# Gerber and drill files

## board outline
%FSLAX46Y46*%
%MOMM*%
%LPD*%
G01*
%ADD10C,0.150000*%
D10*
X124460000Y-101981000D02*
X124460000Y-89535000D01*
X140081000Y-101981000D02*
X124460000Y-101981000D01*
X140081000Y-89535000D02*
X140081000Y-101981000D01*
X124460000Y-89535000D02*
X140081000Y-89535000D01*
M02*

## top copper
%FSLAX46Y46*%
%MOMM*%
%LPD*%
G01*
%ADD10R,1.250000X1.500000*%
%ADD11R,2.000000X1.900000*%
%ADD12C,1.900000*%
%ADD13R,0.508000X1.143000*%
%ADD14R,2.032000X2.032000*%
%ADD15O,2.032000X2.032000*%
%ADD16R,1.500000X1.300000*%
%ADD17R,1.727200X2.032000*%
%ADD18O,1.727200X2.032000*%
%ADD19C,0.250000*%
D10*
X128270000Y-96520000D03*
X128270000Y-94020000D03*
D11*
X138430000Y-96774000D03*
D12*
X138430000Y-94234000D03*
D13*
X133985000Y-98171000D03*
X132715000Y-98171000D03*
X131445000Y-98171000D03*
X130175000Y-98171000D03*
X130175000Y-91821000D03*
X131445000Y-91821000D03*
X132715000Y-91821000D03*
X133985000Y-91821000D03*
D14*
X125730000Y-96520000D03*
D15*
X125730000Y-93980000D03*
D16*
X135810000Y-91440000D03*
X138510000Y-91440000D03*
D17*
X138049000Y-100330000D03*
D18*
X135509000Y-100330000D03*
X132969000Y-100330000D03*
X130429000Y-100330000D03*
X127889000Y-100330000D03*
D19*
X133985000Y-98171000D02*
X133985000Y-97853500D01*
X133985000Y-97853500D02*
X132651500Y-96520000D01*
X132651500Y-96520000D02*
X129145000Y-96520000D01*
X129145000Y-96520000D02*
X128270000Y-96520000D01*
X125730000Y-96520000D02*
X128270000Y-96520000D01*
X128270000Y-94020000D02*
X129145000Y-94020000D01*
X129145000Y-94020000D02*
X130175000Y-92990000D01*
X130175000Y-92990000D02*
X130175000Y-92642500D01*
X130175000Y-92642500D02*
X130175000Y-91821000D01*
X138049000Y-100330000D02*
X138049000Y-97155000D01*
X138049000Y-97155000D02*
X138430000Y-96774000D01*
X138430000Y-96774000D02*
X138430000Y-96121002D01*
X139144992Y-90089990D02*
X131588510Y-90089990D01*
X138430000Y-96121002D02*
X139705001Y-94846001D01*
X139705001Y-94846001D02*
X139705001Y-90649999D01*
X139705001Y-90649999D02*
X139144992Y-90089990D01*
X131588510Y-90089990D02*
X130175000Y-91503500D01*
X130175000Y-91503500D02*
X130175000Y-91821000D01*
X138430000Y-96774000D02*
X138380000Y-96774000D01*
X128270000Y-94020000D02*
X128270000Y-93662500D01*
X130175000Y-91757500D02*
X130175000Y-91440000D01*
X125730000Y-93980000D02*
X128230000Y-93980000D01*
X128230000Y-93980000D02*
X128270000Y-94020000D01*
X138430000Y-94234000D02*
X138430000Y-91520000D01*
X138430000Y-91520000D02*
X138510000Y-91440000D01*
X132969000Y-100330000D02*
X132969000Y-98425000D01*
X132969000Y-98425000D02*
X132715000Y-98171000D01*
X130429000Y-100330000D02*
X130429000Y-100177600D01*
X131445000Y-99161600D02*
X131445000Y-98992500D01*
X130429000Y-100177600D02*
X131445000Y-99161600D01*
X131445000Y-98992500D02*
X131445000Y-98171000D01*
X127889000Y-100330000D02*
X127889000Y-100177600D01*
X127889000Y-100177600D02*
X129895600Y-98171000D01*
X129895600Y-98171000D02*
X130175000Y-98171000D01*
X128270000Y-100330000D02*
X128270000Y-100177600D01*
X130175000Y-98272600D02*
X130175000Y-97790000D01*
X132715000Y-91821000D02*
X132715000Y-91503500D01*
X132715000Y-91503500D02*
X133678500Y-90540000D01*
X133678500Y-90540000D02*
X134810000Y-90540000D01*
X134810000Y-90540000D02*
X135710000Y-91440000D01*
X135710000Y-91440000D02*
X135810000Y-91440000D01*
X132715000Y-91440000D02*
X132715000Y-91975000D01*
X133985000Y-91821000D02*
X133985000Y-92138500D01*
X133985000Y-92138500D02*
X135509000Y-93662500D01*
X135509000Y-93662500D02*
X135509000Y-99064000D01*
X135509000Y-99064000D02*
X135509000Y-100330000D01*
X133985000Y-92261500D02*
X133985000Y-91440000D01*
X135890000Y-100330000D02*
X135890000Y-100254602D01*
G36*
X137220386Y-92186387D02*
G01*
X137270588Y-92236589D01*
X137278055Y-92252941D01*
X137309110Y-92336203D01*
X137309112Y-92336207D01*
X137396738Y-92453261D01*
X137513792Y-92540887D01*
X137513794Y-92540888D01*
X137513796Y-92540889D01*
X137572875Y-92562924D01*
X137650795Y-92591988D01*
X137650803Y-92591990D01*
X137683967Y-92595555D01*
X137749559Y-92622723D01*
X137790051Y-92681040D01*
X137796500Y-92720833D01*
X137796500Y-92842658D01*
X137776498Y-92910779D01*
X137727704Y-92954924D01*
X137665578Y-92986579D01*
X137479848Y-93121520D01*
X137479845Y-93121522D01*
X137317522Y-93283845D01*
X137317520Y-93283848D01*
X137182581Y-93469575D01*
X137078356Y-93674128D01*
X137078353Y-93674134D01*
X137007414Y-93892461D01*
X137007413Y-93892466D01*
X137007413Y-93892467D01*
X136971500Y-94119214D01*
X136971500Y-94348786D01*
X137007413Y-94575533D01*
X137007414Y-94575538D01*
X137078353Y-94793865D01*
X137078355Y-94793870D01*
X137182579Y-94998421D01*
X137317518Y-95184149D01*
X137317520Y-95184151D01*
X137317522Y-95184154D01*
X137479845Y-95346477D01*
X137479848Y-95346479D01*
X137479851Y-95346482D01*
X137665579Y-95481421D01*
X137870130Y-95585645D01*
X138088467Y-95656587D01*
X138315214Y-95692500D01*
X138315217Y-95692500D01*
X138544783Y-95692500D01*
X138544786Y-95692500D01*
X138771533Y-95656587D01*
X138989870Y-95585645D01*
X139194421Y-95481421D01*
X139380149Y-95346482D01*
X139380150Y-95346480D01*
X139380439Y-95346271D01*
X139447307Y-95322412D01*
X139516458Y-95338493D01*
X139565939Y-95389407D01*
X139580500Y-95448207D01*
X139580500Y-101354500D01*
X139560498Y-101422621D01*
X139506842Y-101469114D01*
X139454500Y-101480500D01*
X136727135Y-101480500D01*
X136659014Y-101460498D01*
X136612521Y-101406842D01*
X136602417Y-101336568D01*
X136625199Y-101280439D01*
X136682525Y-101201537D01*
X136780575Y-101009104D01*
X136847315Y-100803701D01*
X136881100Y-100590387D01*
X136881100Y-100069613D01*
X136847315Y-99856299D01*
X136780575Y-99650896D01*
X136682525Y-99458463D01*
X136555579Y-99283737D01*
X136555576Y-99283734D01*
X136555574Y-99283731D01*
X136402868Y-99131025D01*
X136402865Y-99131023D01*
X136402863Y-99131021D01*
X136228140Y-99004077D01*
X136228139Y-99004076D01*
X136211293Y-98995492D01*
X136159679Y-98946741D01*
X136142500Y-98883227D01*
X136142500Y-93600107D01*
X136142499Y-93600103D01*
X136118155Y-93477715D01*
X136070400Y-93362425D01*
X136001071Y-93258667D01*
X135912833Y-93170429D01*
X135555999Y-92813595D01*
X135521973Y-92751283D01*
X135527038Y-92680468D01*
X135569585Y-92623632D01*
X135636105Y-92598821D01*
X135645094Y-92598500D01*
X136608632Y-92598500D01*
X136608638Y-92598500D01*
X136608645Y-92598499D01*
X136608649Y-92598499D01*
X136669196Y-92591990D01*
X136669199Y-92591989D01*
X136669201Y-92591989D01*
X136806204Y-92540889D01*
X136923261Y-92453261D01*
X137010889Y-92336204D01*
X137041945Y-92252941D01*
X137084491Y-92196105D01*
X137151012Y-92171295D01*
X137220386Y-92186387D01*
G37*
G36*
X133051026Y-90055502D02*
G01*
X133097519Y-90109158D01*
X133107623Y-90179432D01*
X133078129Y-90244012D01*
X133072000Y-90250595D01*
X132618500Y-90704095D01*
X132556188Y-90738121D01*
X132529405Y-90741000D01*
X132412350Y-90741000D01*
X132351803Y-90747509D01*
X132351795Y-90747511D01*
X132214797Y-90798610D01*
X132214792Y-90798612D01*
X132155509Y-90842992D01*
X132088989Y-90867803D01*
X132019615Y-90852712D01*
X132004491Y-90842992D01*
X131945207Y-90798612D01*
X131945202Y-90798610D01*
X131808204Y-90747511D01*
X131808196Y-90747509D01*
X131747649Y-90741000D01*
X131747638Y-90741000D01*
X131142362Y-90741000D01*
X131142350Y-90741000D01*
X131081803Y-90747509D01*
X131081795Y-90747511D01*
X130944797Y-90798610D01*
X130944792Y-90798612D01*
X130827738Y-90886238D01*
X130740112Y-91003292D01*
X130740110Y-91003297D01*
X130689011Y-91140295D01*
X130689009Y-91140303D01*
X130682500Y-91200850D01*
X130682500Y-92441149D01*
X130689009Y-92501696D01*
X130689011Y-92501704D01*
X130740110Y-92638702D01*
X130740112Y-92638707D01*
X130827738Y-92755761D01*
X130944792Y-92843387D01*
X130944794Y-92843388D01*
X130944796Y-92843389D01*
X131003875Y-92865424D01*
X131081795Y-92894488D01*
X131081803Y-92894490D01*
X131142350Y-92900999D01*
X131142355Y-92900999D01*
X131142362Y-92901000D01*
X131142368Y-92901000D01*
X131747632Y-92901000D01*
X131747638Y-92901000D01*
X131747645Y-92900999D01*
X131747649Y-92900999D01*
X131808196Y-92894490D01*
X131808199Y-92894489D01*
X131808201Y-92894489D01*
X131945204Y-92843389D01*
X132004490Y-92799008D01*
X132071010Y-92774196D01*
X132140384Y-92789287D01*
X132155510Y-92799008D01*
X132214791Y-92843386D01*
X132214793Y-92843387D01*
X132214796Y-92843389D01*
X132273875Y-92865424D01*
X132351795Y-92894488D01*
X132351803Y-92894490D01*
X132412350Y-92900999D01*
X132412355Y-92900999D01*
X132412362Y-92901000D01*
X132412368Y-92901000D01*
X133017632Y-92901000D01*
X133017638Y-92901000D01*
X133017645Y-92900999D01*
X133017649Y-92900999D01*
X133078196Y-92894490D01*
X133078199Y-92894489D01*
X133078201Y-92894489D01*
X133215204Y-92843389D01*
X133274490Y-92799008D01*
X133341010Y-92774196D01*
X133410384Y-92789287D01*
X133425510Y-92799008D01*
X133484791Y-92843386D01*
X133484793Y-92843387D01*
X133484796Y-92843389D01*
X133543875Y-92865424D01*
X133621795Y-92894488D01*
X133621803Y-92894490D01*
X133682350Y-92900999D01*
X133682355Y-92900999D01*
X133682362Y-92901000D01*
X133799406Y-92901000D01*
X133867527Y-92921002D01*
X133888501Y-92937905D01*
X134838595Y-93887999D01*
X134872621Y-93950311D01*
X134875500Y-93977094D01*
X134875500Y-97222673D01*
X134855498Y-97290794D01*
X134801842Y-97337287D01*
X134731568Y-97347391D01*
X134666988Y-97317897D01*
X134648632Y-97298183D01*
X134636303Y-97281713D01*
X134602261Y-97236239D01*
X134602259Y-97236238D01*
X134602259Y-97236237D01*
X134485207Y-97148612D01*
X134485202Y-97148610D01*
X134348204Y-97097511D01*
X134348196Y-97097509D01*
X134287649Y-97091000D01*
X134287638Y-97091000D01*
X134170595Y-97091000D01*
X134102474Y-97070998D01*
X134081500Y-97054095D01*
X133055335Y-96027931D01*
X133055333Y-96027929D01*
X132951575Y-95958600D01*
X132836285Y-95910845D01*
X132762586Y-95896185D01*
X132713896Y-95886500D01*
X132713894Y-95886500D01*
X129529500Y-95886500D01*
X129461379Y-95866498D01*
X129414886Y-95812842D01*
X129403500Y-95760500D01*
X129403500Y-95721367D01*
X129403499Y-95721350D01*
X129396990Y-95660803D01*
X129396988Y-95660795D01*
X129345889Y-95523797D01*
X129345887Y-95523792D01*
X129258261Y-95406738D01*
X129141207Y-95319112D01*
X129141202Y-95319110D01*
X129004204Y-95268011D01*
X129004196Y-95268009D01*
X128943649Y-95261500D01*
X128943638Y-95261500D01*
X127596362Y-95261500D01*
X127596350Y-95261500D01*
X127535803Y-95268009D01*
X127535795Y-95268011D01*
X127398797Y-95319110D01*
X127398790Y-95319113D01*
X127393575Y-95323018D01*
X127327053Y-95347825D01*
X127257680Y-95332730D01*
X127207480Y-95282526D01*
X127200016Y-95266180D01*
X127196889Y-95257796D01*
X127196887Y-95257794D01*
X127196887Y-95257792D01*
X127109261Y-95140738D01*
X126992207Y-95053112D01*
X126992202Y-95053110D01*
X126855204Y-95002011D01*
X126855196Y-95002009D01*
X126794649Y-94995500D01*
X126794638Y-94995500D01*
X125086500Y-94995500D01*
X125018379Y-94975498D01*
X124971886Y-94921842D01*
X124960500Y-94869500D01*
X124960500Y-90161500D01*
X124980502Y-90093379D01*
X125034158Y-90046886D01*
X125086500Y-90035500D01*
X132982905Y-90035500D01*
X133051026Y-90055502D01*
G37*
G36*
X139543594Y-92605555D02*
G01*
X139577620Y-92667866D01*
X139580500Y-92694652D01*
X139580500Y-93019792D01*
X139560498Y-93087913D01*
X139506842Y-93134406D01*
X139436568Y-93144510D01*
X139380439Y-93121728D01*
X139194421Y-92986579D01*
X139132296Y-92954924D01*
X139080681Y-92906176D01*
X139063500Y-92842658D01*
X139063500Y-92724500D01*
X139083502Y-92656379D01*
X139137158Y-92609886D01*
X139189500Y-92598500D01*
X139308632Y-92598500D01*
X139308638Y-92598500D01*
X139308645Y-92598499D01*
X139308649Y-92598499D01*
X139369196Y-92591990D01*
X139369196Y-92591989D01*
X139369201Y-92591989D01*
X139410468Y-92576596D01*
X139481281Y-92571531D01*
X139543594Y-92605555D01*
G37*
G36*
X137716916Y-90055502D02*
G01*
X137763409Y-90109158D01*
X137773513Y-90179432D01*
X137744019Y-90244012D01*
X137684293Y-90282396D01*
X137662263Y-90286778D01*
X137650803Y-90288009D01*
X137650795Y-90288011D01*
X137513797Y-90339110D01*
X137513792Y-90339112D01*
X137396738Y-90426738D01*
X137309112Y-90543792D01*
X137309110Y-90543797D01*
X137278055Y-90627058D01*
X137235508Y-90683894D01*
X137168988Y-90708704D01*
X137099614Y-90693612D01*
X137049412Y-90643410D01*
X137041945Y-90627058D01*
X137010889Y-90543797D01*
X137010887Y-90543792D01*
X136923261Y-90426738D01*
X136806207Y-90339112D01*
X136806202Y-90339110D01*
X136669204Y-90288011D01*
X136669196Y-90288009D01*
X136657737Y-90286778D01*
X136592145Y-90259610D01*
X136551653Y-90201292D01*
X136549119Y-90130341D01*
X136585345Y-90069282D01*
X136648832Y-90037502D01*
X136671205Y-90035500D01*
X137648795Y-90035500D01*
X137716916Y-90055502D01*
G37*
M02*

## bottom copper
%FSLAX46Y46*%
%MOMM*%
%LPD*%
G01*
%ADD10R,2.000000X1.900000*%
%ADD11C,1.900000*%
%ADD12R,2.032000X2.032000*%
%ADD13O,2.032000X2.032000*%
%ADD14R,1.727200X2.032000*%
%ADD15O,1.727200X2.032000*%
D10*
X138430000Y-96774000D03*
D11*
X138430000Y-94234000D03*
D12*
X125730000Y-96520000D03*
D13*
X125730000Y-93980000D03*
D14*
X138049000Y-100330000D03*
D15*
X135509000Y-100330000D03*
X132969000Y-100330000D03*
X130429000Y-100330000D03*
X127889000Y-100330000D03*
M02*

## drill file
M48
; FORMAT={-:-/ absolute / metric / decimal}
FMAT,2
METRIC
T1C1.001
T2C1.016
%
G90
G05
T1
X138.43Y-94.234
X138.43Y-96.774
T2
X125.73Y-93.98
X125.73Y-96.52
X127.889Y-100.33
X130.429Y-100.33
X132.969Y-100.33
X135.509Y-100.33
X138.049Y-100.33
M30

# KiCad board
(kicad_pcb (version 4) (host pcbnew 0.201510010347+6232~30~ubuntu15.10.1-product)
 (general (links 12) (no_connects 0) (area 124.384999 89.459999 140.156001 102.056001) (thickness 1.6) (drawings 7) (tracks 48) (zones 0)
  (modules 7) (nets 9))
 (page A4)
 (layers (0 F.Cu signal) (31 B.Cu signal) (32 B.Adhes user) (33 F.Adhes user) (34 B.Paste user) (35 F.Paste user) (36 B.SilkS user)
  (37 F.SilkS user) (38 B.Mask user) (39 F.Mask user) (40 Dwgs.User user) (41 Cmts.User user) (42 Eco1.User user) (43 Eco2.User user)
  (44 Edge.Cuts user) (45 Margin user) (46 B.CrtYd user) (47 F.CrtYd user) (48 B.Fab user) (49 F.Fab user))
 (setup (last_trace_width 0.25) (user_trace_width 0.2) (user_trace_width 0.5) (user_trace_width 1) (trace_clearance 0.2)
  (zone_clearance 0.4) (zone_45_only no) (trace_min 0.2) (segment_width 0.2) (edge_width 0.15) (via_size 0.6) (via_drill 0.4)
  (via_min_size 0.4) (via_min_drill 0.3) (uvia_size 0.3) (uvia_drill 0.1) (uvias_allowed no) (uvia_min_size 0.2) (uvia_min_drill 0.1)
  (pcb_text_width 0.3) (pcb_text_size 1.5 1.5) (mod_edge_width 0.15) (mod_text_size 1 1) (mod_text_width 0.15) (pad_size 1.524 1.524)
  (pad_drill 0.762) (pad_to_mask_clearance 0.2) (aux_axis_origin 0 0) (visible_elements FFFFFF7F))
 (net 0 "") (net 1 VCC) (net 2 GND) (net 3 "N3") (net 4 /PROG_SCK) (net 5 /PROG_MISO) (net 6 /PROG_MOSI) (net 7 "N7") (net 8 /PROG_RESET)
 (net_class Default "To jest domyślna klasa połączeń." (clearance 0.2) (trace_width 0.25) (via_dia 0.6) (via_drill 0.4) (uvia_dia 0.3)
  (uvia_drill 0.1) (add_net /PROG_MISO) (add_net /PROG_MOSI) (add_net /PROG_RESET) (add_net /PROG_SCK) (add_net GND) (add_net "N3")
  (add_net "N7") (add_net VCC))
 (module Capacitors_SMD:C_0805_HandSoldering (layer F.Cu) (at 128.27 95.27 90)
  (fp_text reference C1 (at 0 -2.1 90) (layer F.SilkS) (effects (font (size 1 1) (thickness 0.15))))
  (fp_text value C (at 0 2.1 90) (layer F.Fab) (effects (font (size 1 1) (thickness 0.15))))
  (pad 1 smd rect (at -1.25 0 90) (size 1.5 1.25) (layers F.Cu F.Paste F.Mask) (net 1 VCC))
  (pad 2 smd rect (at 1.25 0 90) (size 1.5 1.25) (layers F.Cu F.Paste F.Mask) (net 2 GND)))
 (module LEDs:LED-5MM (layer F.Cu) (at 138.43 96.774 90)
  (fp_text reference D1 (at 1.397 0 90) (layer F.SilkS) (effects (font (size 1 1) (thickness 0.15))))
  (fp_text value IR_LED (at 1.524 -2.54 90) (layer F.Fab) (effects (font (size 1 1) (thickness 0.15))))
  (pad 1 thru_hole rect (at 0 0 180) (size 2 1.9) (drill 1.00076) (layers *.Cu *.Mask F.SilkS) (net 2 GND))
  (pad 2 thru_hole circle (at 2.54 0 90) (size 1.9 1.9) (drill 1.00076) (layers *.Cu *.Mask F.SilkS) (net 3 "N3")))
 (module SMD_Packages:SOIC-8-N (layer F.Cu) (at 132.08 94.996 180)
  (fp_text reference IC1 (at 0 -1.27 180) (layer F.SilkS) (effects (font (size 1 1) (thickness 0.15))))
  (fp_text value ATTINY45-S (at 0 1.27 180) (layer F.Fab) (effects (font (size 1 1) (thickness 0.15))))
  (pad 8 smd rect (at -1.905 -3.175 180) (size 0.508 1.143) (layers F.Cu F.Paste F.Mask) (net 1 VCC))
  (pad 7 smd rect (at -0.635 -3.175 180) (size 0.508 1.143) (layers F.Cu F.Paste F.Mask) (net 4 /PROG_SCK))
  (pad 6 smd rect (at 0.635 -3.175 180) (size 0.508 1.143) (layers F.Cu F.Paste F.Mask) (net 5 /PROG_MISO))
  (pad 5 smd rect (at 1.905 -3.175 180) (size 0.508 1.143) (layers F.Cu F.Paste F.Mask) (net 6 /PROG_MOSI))
  (pad 4 smd rect (at 1.905 3.175 180) (size 0.508 1.143) (layers F.Cu F.Paste F.Mask) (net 2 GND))
  (pad 3 smd rect (at 0.635 3.175 180) (size 0.508 1.143) (layers F.Cu F.Paste F.Mask))
  (pad 2 smd rect (at -0.635 3.175 180) (size 0.508 1.143) (layers F.Cu F.Paste F.Mask) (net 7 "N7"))
  (pad 1 smd rect (at -1.905 3.175 180) (size 0.508 1.143) (layers F.Cu F.Paste F.Mask) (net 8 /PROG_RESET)))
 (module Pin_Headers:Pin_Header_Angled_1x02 (layer F.Cu) (at 125.73 96.52 180)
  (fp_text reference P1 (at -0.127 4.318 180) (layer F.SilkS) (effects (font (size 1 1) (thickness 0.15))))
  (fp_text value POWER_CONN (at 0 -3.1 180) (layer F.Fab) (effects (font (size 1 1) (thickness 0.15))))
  (pad 1 thru_hole rect (at 0 0 180) (size 2.032 2.032) (drill 1.016) (layers *.Cu *.Mask F.SilkS) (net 1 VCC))
  (pad 2 thru_hole oval (at 0 2.54 180) (size 2.032 2.032) (drill 1.016) (layers *.Cu *.Mask F.SilkS) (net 2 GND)))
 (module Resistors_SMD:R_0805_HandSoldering (layer F.Cu) (at 137.16 91.44)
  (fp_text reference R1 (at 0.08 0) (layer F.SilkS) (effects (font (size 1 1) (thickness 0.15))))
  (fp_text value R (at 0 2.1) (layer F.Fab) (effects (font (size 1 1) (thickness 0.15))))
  (pad 1 smd rect (at -1.35 0) (size 1.5 1.3) (layers F.Cu F.Paste F.Mask) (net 7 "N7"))
  (pad 2 smd rect (at 1.35 0) (size 1.5 1.3) (layers F.Cu F.Paste F.Mask) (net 3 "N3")))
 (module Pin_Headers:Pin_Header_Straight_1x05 (layer F.Cu) (at 138.049 100.33 270)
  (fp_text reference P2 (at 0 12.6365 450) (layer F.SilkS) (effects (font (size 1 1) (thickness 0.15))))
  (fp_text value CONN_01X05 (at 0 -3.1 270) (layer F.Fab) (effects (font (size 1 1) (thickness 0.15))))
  (pad 1 thru_hole rect (at 0 0 270) (size 2.032 1.7272) (drill 1.016) (layers *.Cu *.Mask F.SilkS) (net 2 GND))
  (pad 2 thru_hole oval (at 0 2.54 270) (size 2.032 1.7272) (drill 1.016) (layers *.Cu *.Mask F.SilkS) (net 8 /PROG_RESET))
  (pad 3 thru_hole oval (at 0 5.08 270) (size 2.032 1.7272) (drill 1.016) (layers *.Cu *.Mask F.SilkS) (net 4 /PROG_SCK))
  (pad 4 thru_hole oval (at 0 7.62 270) (size 2.032 1.7272) (drill 1.016) (layers *.Cu *.Mask F.SilkS) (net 5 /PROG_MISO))
  (pad 5 thru_hole oval (at 0 10.16 270) (size 2.032 1.7272) (drill 1.016) (layers *.Cu *.Mask F.SilkS) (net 6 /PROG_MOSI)))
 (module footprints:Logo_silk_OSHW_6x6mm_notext (layer B.Cu) (at 129.794 92.202)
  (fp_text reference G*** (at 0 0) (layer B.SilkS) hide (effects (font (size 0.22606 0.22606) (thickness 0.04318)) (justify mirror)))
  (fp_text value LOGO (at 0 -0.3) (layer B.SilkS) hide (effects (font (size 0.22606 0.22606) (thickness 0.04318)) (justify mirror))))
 (gr_line (start 124.46 101.981) (end 124.46 89.535) (layer Edge.Cuts) (width 0.15))
 (gr_line (start 140.081 101.981) (end 124.46 101.981) (layer Edge.Cuts) (width 0.15))
 (gr_line (start 140.081 89.535) (end 140.081 101.981) (layer Edge.Cuts) (width 0.15))
 (gr_line (start 124.46 89.535) (end 140.081 89.535) (layer Edge.Cuts) (width 0.15))
 (segment (start 133.985 98.171) (end 133.985 97.8535) (width 0.25) (layer F.Cu) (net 1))
 (segment (start 133.985 97.8535) (end 132.6515 96.52) (width 0.25) (layer F.Cu) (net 1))
 (segment (start 132.6515 96.52) (end 129.145 96.52) (width 0.25) (layer F.Cu) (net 1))
 (segment (start 129.145 96.52) (end 128.27 96.52) (width 0.25) (layer F.Cu) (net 1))
 (segment (start 125.73 96.52) (end 128.27 96.52) (width 0.25) (layer F.Cu) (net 1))
 (segment (start 128.27 94.02) (end 129.145 94.02) (width 0.25) (layer F.Cu) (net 2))
 (segment (start 129.145 94.02) (end 130.175 92.99) (width 0.25) (layer F.Cu) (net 2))
 (segment (start 130.175 92.99) (end 130.175 92.6425) (width 0.25) (layer F.Cu) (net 2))
 (segment (start 130.175 92.6425) (end 130.175 91.821) (width 0.25) (layer F.Cu) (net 2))
 (segment (start 138.049 100.33) (end 138.049 97.155) (width 0.25) (layer F.Cu) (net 2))
 (segment (start 138.049 97.155) (end 138.43 96.774) (width 0.25) (layer F.Cu) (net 2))
 (segment (start 138.43 96.774) (end 138.43 96.121002) (width 0.25) (layer F.Cu) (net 2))
 (segment (start 139.144992 90.08999) (end 131.58851 90.08999) (width 0.25) (layer F.Cu) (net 2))
 (segment (start 138.43 96.121002) (end 139.705001 94.846001) (width 0.25) (layer F.Cu) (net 2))
 (segment (start 139.705001 94.846001) (end 139.705001 90.649999) (width 0.25) (layer F.Cu) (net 2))
 (segment (start 139.705001 90.649999) (end 139.144992 90.08999) (width 0.25) (layer F.Cu) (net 2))
 (segment (start 131.58851 90.08999) (end 130.175 91.5035) (width 0.25) (layer F.Cu) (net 2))
 (segment (start 130.175 91.5035) (end 130.175 91.821) (width 0.25) (layer F.Cu) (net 2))
 (segment (start 138.43 96.774) (end 138.38 96.774) (width 0.25) (layer F.Cu) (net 2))
 (segment (start 128.27 94.02) (end 128.27 93.6625) (width 0.25) (layer F.Cu) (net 2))
 (segment (start 130.175 91.7575) (end 130.175 91.44) (width 0.25) (layer F.Cu) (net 2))
 (segment (start 125.73 93.98) (end 128.23 93.98) (width 0.25) (layer F.Cu) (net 2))
 (segment (start 128.23 93.98) (end 128.27 94.02) (width 0.25) (layer F.Cu) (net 2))
 (segment (start 138.43 94.234) (end 138.43 91.52) (width 0.25) (layer F.Cu) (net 3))
 (segment (start 138.43 91.52) (end 138.51 91.44) (width 0.25) (layer F.Cu) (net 3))
 (segment (start 132.969 100.33) (end 132.969 98.425) (width 0.25) (layer F.Cu) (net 4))
 (segment (start 132.969 98.425) (end 132.715 98.171) (width 0.25) (layer F.Cu) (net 4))
 (segment (start 130.429 100.33) (end 130.429 100.1776) (width 0.25) (layer F.Cu) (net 5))
 (segment (start 131.445 99.1616) (end 131.445 98.9925) (width 0.25) (layer F.Cu) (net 5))
 (segment (start 130.429 100.1776) (end 131.445 99.1616) (width 0.25) (layer F.Cu) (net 5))
 (segment (start 131.445 98.9925) (end 131.445 98.171) (width 0.25) (layer F.Cu) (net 5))
 (segment (start 127.889 100.33) (end 127.889 100.1776) (width 0.25) (layer F.Cu) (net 6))
 (segment (start 127.889 100.1776) (end 129.8956 98.171) (width 0.25) (layer F.Cu) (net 6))
 (segment (start 129.8956 98.171) (end 130.175 98.171) (width 0.25) (layer F.Cu) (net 6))
 (segment (start 128.27 100.33) (end 128.27 100.1776) (width 0.25) (layer F.Cu) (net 6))
 (segment (start 130.175 98.2726) (end 130.175 97.79) (width 0.25) (layer F.Cu) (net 6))
 (segment (start 132.715 91.821) (end 132.715 91.5035) (width 0.25) (layer F.Cu) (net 7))
 (segment (start 132.715 91.5035) (end 133.6785 90.54) (width 0.25) (layer F.Cu) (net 7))
 (segment (start 133.6785 90.54) (end 134.81 90.54) (width 0.25) (layer F.Cu) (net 7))
 (segment (start 134.81 90.54) (end 135.71 91.44) (width 0.25) (layer F.Cu) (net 7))
 (segment (start 135.71 91.44) (end 135.81 91.44) (width 0.25) (layer F.Cu) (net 7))
 (segment (start 132.715 91.44) (end 132.715 91.975) (width 0.25) (layer F.Cu) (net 7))
 (segment (start 133.985 91.821) (end 133.985 92.1385) (width 0.25) (layer F.Cu) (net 8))
 (segment (start 133.985 92.1385) (end 135.509 93.6625) (width 0.25) (layer F.Cu) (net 8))
 (segment (start 135.509 93.6625) (end 135.509 99.064) (width 0.25) (layer F.Cu) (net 8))
 (segment (start 135.509 99.064) (end 135.509 100.33) (width 0.25) (layer F.Cu) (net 8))
 (segment (start 133.985 92.2615) (end 133.985 91.44) (width 0.25) (layer F.Cu) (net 8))
 (segment (start 135.89 100.33) (end 135.89 100.254602) (width 0.25) (layer F.Cu) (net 8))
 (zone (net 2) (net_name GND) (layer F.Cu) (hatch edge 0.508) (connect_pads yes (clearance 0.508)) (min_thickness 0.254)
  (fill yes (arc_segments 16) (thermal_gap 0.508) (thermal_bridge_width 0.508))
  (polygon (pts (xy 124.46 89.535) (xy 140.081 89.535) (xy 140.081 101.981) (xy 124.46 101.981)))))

